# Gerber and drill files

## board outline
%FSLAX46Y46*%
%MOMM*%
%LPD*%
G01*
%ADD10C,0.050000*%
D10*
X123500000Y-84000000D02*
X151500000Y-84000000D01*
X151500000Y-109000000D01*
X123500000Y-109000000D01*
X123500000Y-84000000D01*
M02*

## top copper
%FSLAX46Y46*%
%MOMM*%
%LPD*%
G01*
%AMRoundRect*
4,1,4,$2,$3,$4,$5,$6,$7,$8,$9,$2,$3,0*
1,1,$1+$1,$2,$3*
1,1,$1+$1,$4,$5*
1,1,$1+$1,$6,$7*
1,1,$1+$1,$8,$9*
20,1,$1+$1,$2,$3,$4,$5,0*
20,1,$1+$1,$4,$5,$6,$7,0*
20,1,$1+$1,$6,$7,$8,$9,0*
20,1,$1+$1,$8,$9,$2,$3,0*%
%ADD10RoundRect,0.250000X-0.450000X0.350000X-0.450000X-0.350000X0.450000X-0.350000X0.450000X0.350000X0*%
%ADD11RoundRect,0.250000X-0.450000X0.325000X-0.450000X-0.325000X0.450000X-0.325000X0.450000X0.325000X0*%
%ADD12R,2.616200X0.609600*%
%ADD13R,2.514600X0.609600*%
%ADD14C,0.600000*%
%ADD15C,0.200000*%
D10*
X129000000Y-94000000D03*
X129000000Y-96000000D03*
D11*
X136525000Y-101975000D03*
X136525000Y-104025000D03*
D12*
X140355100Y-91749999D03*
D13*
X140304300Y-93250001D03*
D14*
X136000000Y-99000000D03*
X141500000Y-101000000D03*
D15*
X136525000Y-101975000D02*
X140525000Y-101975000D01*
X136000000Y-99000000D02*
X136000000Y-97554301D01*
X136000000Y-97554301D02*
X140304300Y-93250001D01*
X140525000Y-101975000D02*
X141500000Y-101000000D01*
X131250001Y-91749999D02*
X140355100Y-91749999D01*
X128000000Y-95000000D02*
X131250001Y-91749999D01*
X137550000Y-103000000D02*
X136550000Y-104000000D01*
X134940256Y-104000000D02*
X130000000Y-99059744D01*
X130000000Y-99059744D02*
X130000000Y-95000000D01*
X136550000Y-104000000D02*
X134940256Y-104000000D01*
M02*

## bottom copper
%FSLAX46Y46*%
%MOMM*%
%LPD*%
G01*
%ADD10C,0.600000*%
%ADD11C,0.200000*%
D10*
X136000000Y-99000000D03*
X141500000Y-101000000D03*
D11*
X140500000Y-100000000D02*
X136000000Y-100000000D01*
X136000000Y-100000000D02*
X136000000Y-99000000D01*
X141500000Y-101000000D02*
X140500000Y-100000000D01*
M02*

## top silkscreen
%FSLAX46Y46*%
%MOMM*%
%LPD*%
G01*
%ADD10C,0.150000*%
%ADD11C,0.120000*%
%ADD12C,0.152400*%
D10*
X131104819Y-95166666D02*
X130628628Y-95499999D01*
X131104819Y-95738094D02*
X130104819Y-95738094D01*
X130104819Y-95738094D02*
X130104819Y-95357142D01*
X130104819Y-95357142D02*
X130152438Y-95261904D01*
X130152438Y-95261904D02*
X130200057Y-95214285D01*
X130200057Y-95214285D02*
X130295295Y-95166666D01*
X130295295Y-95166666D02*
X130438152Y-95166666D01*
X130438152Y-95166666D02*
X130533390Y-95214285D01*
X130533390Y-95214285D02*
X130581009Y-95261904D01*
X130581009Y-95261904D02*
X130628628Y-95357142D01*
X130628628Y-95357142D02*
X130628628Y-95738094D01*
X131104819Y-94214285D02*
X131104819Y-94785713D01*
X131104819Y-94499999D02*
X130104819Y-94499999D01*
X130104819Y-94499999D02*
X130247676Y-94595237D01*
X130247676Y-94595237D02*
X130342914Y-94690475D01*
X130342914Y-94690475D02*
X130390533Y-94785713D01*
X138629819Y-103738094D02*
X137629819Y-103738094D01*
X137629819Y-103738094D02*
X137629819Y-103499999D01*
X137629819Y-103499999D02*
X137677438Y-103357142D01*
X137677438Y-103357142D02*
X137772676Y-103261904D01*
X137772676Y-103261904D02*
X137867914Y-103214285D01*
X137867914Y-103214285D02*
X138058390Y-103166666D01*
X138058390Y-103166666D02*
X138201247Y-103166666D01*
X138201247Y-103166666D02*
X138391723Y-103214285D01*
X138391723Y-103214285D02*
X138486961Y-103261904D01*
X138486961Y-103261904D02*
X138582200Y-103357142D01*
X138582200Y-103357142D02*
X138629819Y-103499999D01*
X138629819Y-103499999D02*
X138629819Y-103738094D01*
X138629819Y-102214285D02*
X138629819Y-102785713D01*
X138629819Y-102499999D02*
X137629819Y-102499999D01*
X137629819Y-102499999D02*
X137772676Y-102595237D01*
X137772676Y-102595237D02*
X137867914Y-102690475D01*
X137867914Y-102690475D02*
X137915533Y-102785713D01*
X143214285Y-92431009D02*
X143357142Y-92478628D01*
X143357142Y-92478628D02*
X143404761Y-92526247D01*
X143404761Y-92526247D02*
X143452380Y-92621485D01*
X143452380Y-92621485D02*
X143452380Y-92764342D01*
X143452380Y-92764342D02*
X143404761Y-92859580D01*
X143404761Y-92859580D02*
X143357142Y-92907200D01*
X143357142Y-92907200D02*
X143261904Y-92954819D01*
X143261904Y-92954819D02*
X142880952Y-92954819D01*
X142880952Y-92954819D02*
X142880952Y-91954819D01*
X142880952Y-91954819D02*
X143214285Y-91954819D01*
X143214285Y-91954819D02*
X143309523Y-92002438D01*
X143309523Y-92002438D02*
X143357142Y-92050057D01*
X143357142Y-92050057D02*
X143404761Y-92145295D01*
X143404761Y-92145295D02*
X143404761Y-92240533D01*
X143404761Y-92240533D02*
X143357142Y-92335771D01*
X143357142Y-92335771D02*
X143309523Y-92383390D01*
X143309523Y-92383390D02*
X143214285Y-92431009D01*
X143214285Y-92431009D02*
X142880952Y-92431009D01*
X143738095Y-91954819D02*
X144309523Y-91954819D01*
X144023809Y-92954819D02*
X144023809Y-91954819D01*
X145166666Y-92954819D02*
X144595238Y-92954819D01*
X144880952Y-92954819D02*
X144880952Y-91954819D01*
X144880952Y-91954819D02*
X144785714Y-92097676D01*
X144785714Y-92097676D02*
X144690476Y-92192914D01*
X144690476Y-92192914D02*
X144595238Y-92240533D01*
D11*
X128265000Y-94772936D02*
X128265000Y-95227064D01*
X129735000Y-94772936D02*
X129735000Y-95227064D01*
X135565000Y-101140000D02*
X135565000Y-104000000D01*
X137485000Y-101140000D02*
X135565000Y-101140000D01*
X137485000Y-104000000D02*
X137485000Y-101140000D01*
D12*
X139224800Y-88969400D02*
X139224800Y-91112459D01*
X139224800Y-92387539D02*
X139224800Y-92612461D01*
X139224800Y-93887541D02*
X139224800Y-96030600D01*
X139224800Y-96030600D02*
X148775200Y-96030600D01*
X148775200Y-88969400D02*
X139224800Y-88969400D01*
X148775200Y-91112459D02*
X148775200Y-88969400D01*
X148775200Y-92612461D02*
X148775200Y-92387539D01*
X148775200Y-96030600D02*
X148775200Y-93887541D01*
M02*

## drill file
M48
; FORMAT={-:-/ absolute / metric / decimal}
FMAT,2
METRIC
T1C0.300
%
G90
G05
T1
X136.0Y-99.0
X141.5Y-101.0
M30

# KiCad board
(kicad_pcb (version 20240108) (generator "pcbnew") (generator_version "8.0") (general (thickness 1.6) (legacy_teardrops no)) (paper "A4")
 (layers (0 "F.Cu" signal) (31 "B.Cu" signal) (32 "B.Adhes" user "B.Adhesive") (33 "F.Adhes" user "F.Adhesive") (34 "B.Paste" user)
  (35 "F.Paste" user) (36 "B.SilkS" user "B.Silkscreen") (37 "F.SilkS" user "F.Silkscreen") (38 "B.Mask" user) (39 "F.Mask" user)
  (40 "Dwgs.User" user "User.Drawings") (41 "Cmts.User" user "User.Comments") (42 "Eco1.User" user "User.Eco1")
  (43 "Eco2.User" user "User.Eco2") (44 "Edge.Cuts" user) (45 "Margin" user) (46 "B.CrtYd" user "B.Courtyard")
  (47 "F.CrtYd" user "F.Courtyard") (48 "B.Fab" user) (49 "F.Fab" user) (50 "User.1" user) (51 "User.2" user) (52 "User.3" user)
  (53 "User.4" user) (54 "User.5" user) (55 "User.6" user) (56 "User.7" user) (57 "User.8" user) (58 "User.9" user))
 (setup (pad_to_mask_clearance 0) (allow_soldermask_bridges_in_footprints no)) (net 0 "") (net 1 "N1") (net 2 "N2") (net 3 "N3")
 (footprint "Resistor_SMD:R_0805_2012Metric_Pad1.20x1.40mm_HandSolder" (layer "F.Cu") (at 129 95 -90)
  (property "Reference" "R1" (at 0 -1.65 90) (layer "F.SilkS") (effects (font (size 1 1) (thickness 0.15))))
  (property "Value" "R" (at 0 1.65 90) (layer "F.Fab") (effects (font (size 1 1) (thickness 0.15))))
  (fp_line (start -0.227064 0.735) (end 0.227064 0.735) (stroke (width 0.12) (type solid)) (layer "F.SilkS"))
  (fp_line (start -0.227064 -0.735) (end 0.227064 -0.735) (stroke (width 0.12) (type solid)) (layer "F.SilkS"))
  (pad "1" smd roundrect (at -1 0 270) (size 1.2 1.4) (layers "F.Cu" "F.Paste" "F.Mask") (roundrect_rratio 0.208333) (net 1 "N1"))
  (pad "2" smd roundrect (at 1 0 270) (size 1.2 1.4) (layers "F.Cu" "F.Paste" "F.Mask") (roundrect_rratio 0.208333) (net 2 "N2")))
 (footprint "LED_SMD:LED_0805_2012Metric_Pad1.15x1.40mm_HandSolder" (layer "F.Cu") (at 136.525 103 -90)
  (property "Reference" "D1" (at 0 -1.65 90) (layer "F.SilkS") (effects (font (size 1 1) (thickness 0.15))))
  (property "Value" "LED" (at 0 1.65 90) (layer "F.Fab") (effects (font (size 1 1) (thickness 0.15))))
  (fp_line (start -1.86 0.96) (end 1 0.96) (stroke (width 0.12) (type solid)) (layer "F.SilkS"))
  (fp_line (start -1.86 -0.96) (end -1.86 0.96) (stroke (width 0.12) (type solid)) (layer "F.SilkS"))
  (fp_line (start 1 -0.96) (end -1.86 -0.96) (stroke (width 0.12) (type solid)) (layer "F.SilkS"))
  (pad "1" smd roundrect (at -1.025 0 270) (size 1.15 1.4) (layers "F.Cu" "F.Paste" "F.Mask") (roundrect_rratio 0.217391) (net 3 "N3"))
  (pad "2" smd roundrect (at 1.025 0 270) (size 1.15 1.4) (layers "F.Cu" "F.Paste" "F.Mask") (roundrect_rratio 0.217391) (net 2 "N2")))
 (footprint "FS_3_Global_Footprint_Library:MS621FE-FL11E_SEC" (layer "F.Cu") (at 144 92.5)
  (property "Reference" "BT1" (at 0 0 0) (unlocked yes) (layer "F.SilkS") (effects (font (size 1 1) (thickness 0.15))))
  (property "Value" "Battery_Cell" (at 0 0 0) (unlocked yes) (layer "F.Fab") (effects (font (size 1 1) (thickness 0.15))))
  (fp_line (start -4.7752 -3.5306) (end -4.7752 -1.387541) (stroke (width 0.1524) (type solid)) (layer "F.SilkS"))
  (fp_line (start -4.7752 -0.112461) (end -4.7752 0.112461) (stroke (width 0.1524) (type solid)) (layer "F.SilkS"))
  (fp_line (start -4.7752 1.387541) (end -4.7752 3.5306) (stroke (width 0.1524) (type solid)) (layer "F.SilkS"))
  (fp_line (start -4.7752 3.5306) (end 4.7752 3.5306) (stroke (width 0.1524) (type solid)) (layer "F.SilkS"))
  (fp_line (start 4.7752 -3.5306) (end -4.7752 -3.5306) (stroke (width 0.1524) (type solid)) (layer "F.SilkS"))
  (fp_line (start 4.7752 -1.387541) (end 4.7752 -3.5306) (stroke (width 0.1524) (type solid)) (layer "F.SilkS"))
  (fp_line (start 4.7752 0.112461) (end 4.7752 -0.112461) (stroke (width 0.1524) (type solid)) (layer "F.SilkS"))
  (fp_line (start 4.7752 3.5306) (end 4.7752 1.387541) (stroke (width 0.1524) (type solid)) (layer "F.SilkS"))
  (pad "1" smd rect (at -3.6449 -0.750001) (size 2.6162 0.6096) (layers "F.Cu" "F.Paste" "F.Mask") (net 1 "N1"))
  (pad "2" smd rect (at -3.6957 0.750001) (size 2.5146 0.6096) (layers "F.Cu" "F.Paste" "F.Mask") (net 3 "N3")))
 (gr_rect (start 123.5 84) (end 151.5 109) (stroke (width 0.05) (type default)) (fill none) (layer "Edge.Cuts"))
 (segment (start 136.525 101.975) (end 140.525 101.975) (width 0.2) (layer "F.Cu") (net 3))
 (segment (start 136 99) (end 136 97.554301) (width 0.2) (layer "F.Cu") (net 3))
 (segment (start 136 97.554301) (end 140.3043 93.250001) (width 0.2) (layer "F.Cu") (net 3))
 (segment (start 140.525 101.975) (end 141.5 101) (width 0.2) (layer "F.Cu") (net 3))
 (via (at 136 99) (size 0.6) (drill 0.3) (layers "F.Cu" "B.Cu") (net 3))
 (via (at 141.5 101) (size 0.6) (drill 0.3) (layers "F.Cu" "B.Cu") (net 3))
 (segment (start 140.5 100) (end 136 100) (width 0.2) (layer "B.Cu") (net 3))
 (segment (start 136 100) (end 136 99) (width 0.2) (layer "B.Cu") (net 3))
 (segment (start 141.5 101) (end 140.5 100) (width 0.2) (layer "B.Cu") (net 3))
 (segment (start 131.250001 91.749999) (end 140.3551 91.749999) (width 0.2) (layer "F.Cu") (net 1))
 (segment (start 128 95) (end 131.250001 91.749999) (width 0.2) (layer "F.Cu") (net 1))
 (segment (start 137.55 103) (end 136.55 104) (width 0.2) (layer "F.Cu") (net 2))
 (segment (start 134.940256 104) (end 130 99.059744) (width 0.2) (layer "F.Cu") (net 2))
 (segment (start 130 99.059744) (end 130 95) (width 0.2) (layer "F.Cu") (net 2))
 (segment (start 136.55 104) (end 134.940256 104) (width 0.2) (layer "F.Cu") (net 2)))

